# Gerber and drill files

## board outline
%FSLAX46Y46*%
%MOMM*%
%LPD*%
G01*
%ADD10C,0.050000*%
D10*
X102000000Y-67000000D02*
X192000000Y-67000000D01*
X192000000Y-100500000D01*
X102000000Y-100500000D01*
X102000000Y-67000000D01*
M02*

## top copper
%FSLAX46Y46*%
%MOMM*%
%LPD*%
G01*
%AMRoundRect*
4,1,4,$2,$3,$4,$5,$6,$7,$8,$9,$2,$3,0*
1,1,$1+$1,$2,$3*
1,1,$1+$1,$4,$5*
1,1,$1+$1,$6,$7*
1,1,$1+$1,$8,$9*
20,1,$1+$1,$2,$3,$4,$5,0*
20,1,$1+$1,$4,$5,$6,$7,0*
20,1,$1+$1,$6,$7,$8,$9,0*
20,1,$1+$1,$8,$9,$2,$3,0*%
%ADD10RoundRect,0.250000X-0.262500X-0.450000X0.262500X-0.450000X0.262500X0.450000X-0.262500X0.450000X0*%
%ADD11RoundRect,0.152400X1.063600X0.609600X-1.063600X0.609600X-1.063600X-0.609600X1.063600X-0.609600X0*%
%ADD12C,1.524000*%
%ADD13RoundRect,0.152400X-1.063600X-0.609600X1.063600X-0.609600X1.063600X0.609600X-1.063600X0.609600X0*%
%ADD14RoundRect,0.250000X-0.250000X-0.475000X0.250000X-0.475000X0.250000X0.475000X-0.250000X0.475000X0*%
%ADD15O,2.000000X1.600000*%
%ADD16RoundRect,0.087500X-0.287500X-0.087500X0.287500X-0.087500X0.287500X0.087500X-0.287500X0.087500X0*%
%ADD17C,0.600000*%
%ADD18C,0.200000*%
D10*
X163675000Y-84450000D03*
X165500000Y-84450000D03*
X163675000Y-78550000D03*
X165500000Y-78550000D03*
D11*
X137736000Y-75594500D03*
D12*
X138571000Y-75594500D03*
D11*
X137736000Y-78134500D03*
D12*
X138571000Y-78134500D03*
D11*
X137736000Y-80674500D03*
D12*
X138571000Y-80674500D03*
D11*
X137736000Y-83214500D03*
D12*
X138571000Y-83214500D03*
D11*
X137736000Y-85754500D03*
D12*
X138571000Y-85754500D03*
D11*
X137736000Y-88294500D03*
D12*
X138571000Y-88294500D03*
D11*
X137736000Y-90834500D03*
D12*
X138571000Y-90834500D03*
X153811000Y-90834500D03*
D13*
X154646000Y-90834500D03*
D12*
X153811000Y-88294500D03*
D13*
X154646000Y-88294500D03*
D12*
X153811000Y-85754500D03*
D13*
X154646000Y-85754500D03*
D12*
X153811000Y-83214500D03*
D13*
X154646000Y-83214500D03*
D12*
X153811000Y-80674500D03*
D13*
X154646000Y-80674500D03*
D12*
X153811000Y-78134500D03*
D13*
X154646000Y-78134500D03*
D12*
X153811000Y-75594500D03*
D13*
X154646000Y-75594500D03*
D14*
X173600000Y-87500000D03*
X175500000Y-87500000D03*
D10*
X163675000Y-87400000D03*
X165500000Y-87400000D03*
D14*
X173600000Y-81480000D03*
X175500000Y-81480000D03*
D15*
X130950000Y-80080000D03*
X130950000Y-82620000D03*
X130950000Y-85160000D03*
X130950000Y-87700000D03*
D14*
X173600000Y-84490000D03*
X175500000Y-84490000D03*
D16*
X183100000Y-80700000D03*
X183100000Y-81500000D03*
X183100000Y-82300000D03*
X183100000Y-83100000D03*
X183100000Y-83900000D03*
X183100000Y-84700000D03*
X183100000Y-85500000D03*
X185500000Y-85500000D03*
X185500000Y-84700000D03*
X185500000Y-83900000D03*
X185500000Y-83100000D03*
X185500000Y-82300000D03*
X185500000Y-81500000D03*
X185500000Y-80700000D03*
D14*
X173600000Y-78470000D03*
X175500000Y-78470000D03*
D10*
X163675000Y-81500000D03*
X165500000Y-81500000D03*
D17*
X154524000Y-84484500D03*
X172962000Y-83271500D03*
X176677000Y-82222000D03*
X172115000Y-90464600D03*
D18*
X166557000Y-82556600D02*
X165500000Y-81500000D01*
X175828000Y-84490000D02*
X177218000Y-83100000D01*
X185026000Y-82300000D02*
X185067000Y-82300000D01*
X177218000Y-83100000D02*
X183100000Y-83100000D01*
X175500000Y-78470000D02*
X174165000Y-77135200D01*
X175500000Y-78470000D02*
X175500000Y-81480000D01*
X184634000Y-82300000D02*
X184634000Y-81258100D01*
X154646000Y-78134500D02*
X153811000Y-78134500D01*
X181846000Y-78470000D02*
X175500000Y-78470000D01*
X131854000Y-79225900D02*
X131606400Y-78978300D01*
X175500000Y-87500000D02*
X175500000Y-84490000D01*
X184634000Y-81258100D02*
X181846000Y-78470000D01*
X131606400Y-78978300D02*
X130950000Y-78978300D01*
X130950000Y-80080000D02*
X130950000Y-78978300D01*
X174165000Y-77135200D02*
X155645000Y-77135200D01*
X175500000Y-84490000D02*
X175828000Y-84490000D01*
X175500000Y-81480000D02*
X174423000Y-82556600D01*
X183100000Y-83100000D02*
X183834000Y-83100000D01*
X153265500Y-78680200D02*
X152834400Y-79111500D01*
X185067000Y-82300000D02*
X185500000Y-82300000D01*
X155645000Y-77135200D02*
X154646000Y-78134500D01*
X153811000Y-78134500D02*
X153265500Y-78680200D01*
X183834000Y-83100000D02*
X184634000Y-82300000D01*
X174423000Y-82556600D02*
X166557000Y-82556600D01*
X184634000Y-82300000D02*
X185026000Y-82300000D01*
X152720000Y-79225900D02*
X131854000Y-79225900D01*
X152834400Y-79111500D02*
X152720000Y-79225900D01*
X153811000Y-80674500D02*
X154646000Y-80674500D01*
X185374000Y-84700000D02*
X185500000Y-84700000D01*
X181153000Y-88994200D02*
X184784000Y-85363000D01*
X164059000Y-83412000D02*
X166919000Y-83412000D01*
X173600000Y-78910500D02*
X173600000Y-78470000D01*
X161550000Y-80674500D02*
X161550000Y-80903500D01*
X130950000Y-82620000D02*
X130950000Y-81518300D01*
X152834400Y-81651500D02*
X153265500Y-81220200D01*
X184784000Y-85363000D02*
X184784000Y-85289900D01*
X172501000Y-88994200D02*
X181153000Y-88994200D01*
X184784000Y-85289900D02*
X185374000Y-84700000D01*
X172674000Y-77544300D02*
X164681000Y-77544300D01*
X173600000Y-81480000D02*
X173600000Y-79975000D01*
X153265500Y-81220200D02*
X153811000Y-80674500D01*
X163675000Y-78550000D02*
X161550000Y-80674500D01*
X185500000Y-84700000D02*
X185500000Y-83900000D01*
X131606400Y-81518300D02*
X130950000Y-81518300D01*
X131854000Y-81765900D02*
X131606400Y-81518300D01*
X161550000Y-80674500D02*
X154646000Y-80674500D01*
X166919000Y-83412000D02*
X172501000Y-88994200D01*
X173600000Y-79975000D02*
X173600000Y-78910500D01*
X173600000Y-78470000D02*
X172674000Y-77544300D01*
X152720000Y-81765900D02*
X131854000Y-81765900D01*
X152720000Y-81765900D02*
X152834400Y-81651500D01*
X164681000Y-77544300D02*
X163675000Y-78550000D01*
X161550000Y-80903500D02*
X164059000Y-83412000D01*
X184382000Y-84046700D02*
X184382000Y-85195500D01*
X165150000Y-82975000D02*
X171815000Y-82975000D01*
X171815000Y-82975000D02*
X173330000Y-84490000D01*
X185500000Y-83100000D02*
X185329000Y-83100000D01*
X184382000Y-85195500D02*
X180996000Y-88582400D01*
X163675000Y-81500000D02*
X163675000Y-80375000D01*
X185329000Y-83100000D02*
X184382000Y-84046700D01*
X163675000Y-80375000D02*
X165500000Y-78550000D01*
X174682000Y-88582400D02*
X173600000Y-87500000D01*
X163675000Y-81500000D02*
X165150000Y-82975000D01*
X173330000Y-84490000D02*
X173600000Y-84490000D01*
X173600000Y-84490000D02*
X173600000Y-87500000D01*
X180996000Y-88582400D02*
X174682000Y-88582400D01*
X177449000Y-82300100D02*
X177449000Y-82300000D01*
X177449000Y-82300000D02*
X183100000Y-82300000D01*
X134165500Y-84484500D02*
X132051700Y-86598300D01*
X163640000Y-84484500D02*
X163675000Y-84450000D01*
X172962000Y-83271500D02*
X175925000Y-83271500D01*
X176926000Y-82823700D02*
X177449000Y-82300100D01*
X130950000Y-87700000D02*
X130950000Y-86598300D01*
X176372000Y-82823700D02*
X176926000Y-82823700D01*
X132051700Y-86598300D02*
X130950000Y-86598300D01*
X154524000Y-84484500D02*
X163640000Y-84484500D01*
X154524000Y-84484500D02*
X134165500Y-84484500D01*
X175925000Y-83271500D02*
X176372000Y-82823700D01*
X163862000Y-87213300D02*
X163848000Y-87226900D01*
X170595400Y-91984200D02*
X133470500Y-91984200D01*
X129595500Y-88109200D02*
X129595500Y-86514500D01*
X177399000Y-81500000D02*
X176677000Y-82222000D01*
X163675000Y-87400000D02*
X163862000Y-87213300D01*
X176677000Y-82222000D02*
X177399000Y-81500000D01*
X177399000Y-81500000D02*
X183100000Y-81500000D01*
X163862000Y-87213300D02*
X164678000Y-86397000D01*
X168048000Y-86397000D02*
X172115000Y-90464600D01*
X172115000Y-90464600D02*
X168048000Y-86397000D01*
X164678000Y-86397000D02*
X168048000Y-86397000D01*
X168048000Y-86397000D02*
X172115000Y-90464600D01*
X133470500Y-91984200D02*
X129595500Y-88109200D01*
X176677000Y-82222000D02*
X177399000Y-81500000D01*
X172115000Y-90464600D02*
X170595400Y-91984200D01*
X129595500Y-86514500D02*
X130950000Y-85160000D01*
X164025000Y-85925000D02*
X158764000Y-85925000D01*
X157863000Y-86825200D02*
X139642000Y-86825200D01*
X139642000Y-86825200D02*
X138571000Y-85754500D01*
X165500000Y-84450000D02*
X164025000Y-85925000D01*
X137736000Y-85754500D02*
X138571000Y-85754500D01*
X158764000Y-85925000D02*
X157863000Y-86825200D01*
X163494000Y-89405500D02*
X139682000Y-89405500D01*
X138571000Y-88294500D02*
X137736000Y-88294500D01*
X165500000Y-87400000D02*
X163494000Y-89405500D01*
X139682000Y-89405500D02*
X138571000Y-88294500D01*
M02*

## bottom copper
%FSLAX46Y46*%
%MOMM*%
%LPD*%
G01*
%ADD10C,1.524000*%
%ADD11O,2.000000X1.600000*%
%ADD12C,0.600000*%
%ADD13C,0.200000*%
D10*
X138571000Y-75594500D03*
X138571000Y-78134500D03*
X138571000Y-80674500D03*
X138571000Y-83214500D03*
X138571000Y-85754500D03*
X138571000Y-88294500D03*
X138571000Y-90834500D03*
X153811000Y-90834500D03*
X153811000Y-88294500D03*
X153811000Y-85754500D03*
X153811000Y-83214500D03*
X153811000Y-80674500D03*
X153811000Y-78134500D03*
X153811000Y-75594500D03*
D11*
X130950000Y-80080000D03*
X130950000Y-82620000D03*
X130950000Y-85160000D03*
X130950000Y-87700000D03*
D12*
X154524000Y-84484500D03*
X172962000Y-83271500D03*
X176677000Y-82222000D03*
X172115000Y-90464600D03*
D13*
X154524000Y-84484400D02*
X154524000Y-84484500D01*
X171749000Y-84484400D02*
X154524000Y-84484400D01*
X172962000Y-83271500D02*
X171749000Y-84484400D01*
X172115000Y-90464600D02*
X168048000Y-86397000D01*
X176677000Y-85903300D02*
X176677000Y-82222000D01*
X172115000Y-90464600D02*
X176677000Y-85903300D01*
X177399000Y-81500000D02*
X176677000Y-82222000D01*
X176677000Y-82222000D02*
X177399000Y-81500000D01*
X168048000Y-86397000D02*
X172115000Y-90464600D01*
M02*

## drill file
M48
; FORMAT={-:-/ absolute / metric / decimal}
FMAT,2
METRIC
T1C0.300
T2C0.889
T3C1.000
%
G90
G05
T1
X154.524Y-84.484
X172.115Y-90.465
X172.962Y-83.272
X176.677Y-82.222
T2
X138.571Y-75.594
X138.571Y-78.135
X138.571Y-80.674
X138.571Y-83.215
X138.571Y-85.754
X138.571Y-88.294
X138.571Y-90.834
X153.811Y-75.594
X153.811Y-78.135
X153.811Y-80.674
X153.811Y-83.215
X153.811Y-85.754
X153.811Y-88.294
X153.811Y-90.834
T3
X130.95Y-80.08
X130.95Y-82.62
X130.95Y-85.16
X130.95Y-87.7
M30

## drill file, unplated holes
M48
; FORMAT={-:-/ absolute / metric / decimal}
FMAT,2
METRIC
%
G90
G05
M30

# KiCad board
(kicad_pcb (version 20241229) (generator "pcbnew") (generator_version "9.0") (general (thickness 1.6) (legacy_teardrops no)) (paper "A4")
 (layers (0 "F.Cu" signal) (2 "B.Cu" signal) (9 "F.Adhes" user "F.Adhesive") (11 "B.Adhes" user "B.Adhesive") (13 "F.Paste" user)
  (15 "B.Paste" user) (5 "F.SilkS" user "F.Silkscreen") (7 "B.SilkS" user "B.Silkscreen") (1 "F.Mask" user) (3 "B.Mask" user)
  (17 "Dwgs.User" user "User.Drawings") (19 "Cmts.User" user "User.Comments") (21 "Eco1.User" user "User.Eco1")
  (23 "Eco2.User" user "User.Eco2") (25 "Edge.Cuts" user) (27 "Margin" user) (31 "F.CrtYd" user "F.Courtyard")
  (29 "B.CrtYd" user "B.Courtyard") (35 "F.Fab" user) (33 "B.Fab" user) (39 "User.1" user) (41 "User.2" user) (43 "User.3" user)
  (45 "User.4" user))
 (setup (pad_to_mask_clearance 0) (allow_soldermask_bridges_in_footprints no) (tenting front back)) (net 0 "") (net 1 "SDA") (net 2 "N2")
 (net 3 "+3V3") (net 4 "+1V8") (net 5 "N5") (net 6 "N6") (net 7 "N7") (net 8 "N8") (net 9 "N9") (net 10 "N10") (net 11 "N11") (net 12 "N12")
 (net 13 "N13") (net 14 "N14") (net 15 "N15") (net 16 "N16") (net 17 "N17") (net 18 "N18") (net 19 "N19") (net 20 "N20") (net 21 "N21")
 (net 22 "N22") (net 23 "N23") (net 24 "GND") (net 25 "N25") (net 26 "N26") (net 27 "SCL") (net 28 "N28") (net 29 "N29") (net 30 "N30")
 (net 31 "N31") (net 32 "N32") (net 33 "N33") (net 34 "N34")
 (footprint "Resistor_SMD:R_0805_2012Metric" (layer "F.Cu") (at 164.5875 84.45)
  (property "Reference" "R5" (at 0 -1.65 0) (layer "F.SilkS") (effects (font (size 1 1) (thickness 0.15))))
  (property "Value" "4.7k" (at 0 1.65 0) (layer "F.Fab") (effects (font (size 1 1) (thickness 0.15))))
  (pad "1" smd roundrect (at -0.9125 0) (size 1.025 1.4) (layers "F.Cu" "F.Mask" "F.Paste") (roundrect_rratio 0.243902) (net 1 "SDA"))
  (pad "2" smd roundrect (at 0.9125 0) (size 1.025 1.4) (layers "F.Cu" "F.Mask" "F.Paste") (roundrect_rratio 0.243902) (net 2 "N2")))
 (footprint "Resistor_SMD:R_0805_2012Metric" (layer "F.Cu") (at 164.5875 78.55)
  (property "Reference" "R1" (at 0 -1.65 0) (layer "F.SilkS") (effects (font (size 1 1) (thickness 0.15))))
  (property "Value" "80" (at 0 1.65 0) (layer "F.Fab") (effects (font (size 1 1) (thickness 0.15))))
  (pad "1" smd roundrect (at -0.9125 0) (size 1.025 1.4) (layers "F.Cu" "F.Mask" "F.Paste") (roundrect_rratio 0.243902) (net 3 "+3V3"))
  (pad "2" smd roundrect (at 0.9125 0) (size 1.025 1.4) (layers "F.Cu" "F.Mask" "F.Paste") (roundrect_rratio 0.243902) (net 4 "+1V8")))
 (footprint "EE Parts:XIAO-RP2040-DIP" (layer "F.Cu") (at 146.191 83.2145)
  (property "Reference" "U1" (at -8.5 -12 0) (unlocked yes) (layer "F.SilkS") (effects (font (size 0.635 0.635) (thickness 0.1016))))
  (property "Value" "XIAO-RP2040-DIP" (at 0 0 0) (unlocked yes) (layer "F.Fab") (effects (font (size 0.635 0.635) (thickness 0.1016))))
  (pad "1" smd roundrect (at -8.455 -7.62 180) (size 2.432 1.524) (layers "F.Cu" "F.Mask") (roundrect_rratio 0.1) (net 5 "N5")
   (thermal_bridge_angle 45))
  (pad "1" thru_hole circle (at -7.62 -7.62 180) (size 1.524 1.524) (drill 0.889) (layers "*.Cu" "*.Mask") (remove_unused_layers no)
   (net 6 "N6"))
  (pad "2" smd roundrect (at -8.455 -5.08 180) (size 2.432 1.524) (layers "F.Cu" "F.Mask") (roundrect_rratio 0.1) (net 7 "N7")
   (thermal_bridge_angle 45))
  (pad "2" thru_hole circle (at -7.62 -5.08 180) (size 1.524 1.524) (drill 0.889) (layers "*.Cu" "*.Mask") (remove_unused_layers no)
   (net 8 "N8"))
  (pad "3" smd roundrect (at -8.455 -2.54 180) (size 2.432 1.524) (layers "F.Cu" "F.Mask") (roundrect_rratio 0.1) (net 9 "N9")
   (thermal_bridge_angle 45))
  (pad "3" thru_hole circle (at -7.62 -2.54 180) (size 1.524 1.524) (drill 0.889) (layers "*.Cu" "*.Mask") (remove_unused_layers no)
   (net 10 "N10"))
  (pad "4" smd roundrect (at -8.455 0 180) (size 2.432 1.524) (layers "F.Cu" "F.Mask") (roundrect_rratio 0.1) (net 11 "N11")
   (thermal_bridge_angle 45))
  (pad "4" thru_hole circle (at -7.62 0 180) (size 1.524 1.524) (drill 0.889) (layers "*.Cu" "*.Mask") (remove_unused_layers no)
   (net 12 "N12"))
  (pad "5" smd roundrect (at -8.455 2.54 180) (size 2.432 1.524) (layers "F.Cu" "F.Mask") (roundrect_rratio 0.1) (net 2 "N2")
   (thermal_bridge_angle 45))
  (pad "5" thru_hole circle (at -7.62 2.54 180) (size 1.524 1.524) (drill 0.889) (layers "*.Cu" "*.Mask") (remove_unused_layers no)
   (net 2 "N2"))
  (pad "6" smd roundrect (at -8.455 5.08 180) (size 2.432 1.524) (layers "F.Cu" "F.Mask") (roundrect_rratio 0.1) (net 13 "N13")
   (thermal_bridge_angle 45))
  (pad "6" thru_hole circle (at -7.62 5.08 180) (size 1.524 1.524) (drill 0.889) (layers "*.Cu" "*.Mask") (remove_unused_layers no)
   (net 13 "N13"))
  (pad "7" smd roundrect (at -8.455 7.62 180) (size 2.432 1.524) (layers "F.Cu" "F.Mask") (roundrect_rratio 0.1) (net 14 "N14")
   (thermal_bridge_angle 45))
  (pad "7" thru_hole circle (at -7.62 7.62 180) (size 1.524 1.524) (drill 0.889) (layers "*.Cu" "*.Mask") (remove_unused_layers no)
   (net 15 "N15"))
  (pad "8" thru_hole circle (at 7.62 7.62) (size 1.524 1.524) (drill 0.889) (layers "*.Cu" "*.Mask") (remove_unused_layers no)
   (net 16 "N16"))
  (pad "8" smd roundrect (at 8.455 7.62) (size 2.432 1.524) (layers "F.Cu" "F.Mask") (roundrect_rratio 0.1) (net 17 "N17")
   (thermal_bridge_angle 45))
  (pad "9" thru_hole circle (at 7.62 5.08) (size 1.524 1.524) (drill 0.889) (layers "*.Cu" "*.Mask") (remove_unused_layers no)
   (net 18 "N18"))
  (pad "9" smd roundrect (at 8.455 5.08) (size 2.432 1.524) (layers "F.Cu" "F.Mask") (roundrect_rratio 0.1) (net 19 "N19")
   (thermal_bridge_angle 45))
  (pad "10" thru_hole circle (at 7.62 2.54) (size 1.524 1.524) (drill 0.889) (layers "*.Cu" "*.Mask") (remove_unused_layers no)
   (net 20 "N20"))
  (pad "10" smd roundrect (at 8.455 2.54) (size 2.432 1.524) (layers "F.Cu" "F.Mask") (roundrect_rratio 0.1) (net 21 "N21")
   (thermal_bridge_angle 45))
  (pad "11" thru_hole circle (at 7.62 0) (size 1.524 1.524) (drill 0.889) (layers "*.Cu" "*.Mask") (remove_unused_layers no) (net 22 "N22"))
  (pad "11" smd roundrect (at 8.455 0) (size 2.432 1.524) (layers "F.Cu" "F.Mask") (roundrect_rratio 0.1) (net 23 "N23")
   (thermal_bridge_angle 45))
  (pad "12" thru_hole circle (at 7.62 -2.54) (size 1.524 1.524) (drill 0.889) (layers "*.Cu" "*.Mask") (remove_unused_layers no)
   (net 3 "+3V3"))
  (pad "12" smd roundrect (at 8.455 -2.54) (size 2.432 1.524) (layers "F.Cu" "F.Mask") (roundrect_rratio 0.1) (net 3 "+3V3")
   (thermal_bridge_angle 45))
  (pad "13" thru_hole circle (at 7.62 -5.08) (size 1.524 1.524) (drill 0.889) (layers "*.Cu" "*.Mask") (remove_unused_layers no)
   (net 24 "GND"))
  (pad "13" smd roundrect (at 8.455 -5.08) (size 2.432 1.524) (layers "F.Cu" "F.Mask") (roundrect_rratio 0.1) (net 24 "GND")
   (thermal_bridge_angle 45))
  (pad "14" thru_hole circle (at 7.62 -7.62) (size 1.524 1.524) (drill 0.889) (layers "*.Cu" "*.Mask") (remove_unused_layers no)
   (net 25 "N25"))
  (pad "14" smd roundrect (at 8.455 -7.62) (size 2.432 1.524) (layers "F.Cu" "F.Mask") (roundrect_rratio 0.1) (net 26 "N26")
   (thermal_bridge_angle 45)))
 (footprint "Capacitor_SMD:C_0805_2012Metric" (layer "F.Cu") (at 174.55 87.5)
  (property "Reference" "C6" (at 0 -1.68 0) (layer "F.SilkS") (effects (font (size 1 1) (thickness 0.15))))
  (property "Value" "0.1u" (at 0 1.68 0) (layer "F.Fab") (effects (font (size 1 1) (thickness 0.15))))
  (pad "1" smd roundrect (at -0.95 0) (size 1 1.45) (layers "F.Cu" "F.Mask" "F.Paste") (roundrect_rratio 0.25) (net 4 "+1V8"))
  (pad "2" smd roundrect (at 0.95 0) (size 1 1.45) (layers "F.Cu" "F.Mask" "F.Paste") (roundrect_rratio 0.25) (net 24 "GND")))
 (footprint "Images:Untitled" (layer "F.Cu") (at 186.5 95)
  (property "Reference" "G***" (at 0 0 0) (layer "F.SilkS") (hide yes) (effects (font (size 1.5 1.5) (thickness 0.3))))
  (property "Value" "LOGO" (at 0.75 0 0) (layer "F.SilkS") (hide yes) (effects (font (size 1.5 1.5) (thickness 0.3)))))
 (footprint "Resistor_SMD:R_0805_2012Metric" (layer "F.Cu") (at 164.5875 87.4)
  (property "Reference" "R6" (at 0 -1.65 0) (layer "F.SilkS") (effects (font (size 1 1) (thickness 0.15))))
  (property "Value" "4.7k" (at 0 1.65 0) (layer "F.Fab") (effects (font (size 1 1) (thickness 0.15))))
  (pad "1" smd roundrect (at -0.9125 0) (size 1.025 1.4) (layers "F.Cu" "F.Mask" "F.Paste") (roundrect_rratio 0.243902) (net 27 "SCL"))
  (pad "2" smd roundrect (at 0.9125 0) (size 1.025 1.4) (layers "F.Cu" "F.Mask" "F.Paste") (roundrect_rratio 0.243902) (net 13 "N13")))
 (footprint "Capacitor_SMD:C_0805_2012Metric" (layer "F.Cu") (at 174.55 81.48)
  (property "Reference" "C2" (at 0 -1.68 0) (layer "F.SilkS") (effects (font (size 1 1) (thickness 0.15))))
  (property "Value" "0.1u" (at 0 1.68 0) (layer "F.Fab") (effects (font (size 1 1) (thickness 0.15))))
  (pad "1" smd roundrect (at -0.95 0) (size 1 1.45) (layers "F.Cu" "F.Mask" "F.Paste") (roundrect_rratio 0.25) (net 3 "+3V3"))
  (pad "2" smd roundrect (at 0.95 0) (size 1 1.45) (layers "F.Cu" "F.Mask" "F.Paste") (roundrect_rratio 0.25) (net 24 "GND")))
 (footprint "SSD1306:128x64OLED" (layer "F.Cu") (at 120.35 83.7 -90)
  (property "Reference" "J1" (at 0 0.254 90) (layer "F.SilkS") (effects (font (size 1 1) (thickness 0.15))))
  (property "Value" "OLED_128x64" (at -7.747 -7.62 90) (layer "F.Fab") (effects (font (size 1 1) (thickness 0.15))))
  (pad "1" thru_hole oval (at -3.62 -10.6) (size 2 1.6) (drill 1) (layers "*.Cu" "*.Mask") (remove_unused_layers no) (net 24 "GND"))
  (pad "2" thru_hole oval (at -1.08 -10.6) (size 2 1.6) (drill 1) (layers "*.Cu" "*.Mask") (remove_unused_layers no) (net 3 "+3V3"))
  (pad "3" thru_hole oval (at 1.46 -10.6) (size 2 1.6) (drill 1) (layers "*.Cu" "*.Mask") (remove_unused_layers no) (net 27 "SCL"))
  (pad "4" thru_hole oval (at 4 -10.6) (size 2 1.6) (drill 1) (layers "*.Cu" "*.Mask") (remove_unused_layers no) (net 1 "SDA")))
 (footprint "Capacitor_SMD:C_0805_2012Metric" (layer "F.Cu") (at 174.55 84.49)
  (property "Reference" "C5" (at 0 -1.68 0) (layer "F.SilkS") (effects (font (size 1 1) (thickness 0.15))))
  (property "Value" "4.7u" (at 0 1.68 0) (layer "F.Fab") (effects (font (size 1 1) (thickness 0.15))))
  (pad "1" smd roundrect (at -0.95 0) (size 1 1.45) (layers "F.Cu" "F.Mask" "F.Paste") (roundrect_rratio 0.25) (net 4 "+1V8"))
  (pad "2" smd roundrect (at 0.95 0) (size 1 1.45) (layers "F.Cu" "F.Mask" "F.Paste") (roundrect_rratio 0.25) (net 24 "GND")))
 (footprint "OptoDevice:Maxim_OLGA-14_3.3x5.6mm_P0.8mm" (layer "F.Cu") (at 184.3 83.1)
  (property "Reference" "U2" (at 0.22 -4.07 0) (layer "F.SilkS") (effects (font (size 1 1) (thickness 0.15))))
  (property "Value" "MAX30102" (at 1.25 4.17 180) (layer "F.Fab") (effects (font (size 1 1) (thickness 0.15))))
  (pad "1" smd roundrect (at -1.2 -2.4) (size 0.75 0.35) (layers "F.Cu" "F.Mask" "F.Paste") (roundrect_rratio 0.25) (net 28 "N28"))
  (pad "2" smd roundrect (at -1.2 -1.6) (size 0.75 0.35) (layers "F.Cu" "F.Mask" "F.Paste") (roundrect_rratio 0.25) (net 27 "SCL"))
  (pad "3" smd roundrect (at -1.2 -0.8) (size 0.75 0.35) (layers "F.Cu" "F.Mask" "F.Paste") (roundrect_rratio 0.25) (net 1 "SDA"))
  (pad "4" smd roundrect (at -1.2 0) (size 0.75 0.35) (layers "F.Cu" "F.Mask" "F.Paste") (roundrect_rratio 0.25) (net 24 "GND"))
  (pad "5" smd roundrect (at -1.2 0.8) (size 0.75 0.35) (layers "F.Cu" "F.Mask" "F.Paste") (roundrect_rratio 0.25) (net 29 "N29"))
  (pad "6" smd roundrect (at -1.2 1.6) (size 0.75 0.35) (layers "F.Cu" "F.Mask" "F.Paste") (roundrect_rratio 0.25) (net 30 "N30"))
  (pad "7" smd roundrect (at -1.2 2.4) (size 0.75 0.35) (layers "F.Cu" "F.Mask" "F.Paste") (roundrect_rratio 0.25) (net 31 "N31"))
  (pad "8" smd roundrect (at 1.2 2.4) (size 0.75 0.35) (layers "F.Cu" "F.Mask" "F.Paste") (roundrect_rratio 0.25) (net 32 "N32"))
  (pad "9" smd roundrect (at 1.2 1.6) (size 0.75 0.35) (layers "F.Cu" "F.Mask" "F.Paste") (roundrect_rratio 0.25) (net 3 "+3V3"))
  (pad "10" smd roundrect (at 1.2 0.8) (size 0.75 0.35) (layers "F.Cu" "F.Mask" "F.Paste") (roundrect_rratio 0.25) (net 3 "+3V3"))
  (pad "11" smd roundrect (at 1.2 0) (size 0.75 0.35) (layers "F.Cu" "F.Mask" "F.Paste") (roundrect_rratio 0.25) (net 4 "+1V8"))
  (pad "12" smd roundrect (at 1.2 -0.8) (size 0.75 0.35) (layers "F.Cu" "F.Mask" "F.Paste") (roundrect_rratio 0.25) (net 24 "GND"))
  (pad "13" smd roundrect (at 1.2 -1.6) (size 0.75 0.35) (layers "F.Cu" "F.Mask" "F.Paste") (roundrect_rratio 0.25) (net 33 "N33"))
  (pad "14" smd roundrect (at 1.2 -2.4) (size 0.75 0.35) (layers "F.Cu" "F.Mask" "F.Paste") (roundrect_rratio 0.25) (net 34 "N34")))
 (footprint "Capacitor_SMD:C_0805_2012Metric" (layer "F.Cu") (at 174.55 78.47)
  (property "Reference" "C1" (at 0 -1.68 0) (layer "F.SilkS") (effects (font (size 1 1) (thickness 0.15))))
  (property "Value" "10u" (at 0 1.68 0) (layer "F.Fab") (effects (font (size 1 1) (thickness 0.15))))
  (pad "1" smd roundrect (at -0.95 0) (size 1 1.45) (layers "F.Cu" "F.Mask" "F.Paste") (roundrect_rratio 0.25) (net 3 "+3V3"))
  (pad "2" smd roundrect (at 0.95 0) (size 1 1.45) (layers "F.Cu" "F.Mask" "F.Paste") (roundrect_rratio 0.25) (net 24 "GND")))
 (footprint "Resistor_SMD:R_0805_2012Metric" (layer "F.Cu") (at 164.5875 81.5)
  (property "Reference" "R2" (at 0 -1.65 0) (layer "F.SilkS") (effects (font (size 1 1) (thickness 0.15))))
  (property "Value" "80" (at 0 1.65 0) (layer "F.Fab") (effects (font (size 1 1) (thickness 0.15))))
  (pad "1" smd roundrect (at -0.9125 0) (size 1.025 1.4) (layers "F.Cu" "F.Mask" "F.Paste") (roundrect_rratio 0.243902) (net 4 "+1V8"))
  (pad "2" smd roundrect (at 0.9125 0) (size 1.025 1.4) (layers "F.Cu" "F.Mask" "F.Paste") (roundrect_rratio 0.243902) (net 24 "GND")))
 (gr_rect (start 102 67) (end 192 100.5) (stroke (width 0.05) (type default)) (fill no) (layer "Edge.Cuts"))
 (segment (start 166.557 82.5566) (end 165.5 81.5) (width 0.2) (layer "F.Cu") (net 24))
 (segment (start 175.828 84.49) (end 177.218 83.1) (width 0.2) (layer "F.Cu") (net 24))
 (segment (start 185.026 82.3) (end 185.067 82.3) (width 0.2) (layer "F.Cu") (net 24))
 (segment (start 177.218 83.1) (end 183.1 83.1) (width 0.2) (layer "F.Cu") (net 24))
 (segment (start 175.5 78.47) (end 174.165 77.1352) (width 0.2) (layer "F.Cu") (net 24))
 (segment (start 175.5 78.47) (end 175.5 81.48) (width 0.2) (layer "F.Cu") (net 24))
 (segment (start 184.634 82.3) (end 184.634 81.2581) (width 0.2) (layer "F.Cu") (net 24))
 (segment (start 154.646 78.1345) (end 153.811 78.1345) (width 0.2) (layer "F.Cu") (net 24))
 (segment (start 181.846 78.47) (end 175.5 78.47) (width 0.2) (layer "F.Cu") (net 24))
 (segment (start 131.854 79.2259) (end 131.6064 78.9783) (width 0.2) (layer "F.Cu") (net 24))
 (segment (start 175.5 87.5) (end 175.5 84.49) (width 0.2) (layer "F.Cu") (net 24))
 (segment (start 184.634 81.2581) (end 181.846 78.47) (width 0.2) (layer "F.Cu") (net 24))
 (segment (start 131.6064 78.9783) (end 130.95 78.9783) (width 0.2) (layer "F.Cu") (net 24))
 (segment (start 130.95 80.08) (end 130.95 78.9783) (width 0.2) (layer "F.Cu") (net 24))
 (segment (start 174.165 77.1352) (end 155.645 77.1352) (width 0.2) (layer "F.Cu") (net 24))
 (segment (start 175.5 84.49) (end 175.828 84.49) (width 0.2) (layer "F.Cu") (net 24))
 (segment (start 175.5 81.48) (end 174.423 82.5566) (width 0.2) (layer "F.Cu") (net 24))
 (segment (start 183.1 83.1) (end 183.834 83.1) (width 0.2) (layer "F.Cu") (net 24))
 (segment (start 153.2655 78.6802) (end 152.8344 79.1115) (width 0.2) (layer "F.Cu") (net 24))
 (segment (start 185.067 82.3) (end 185.5 82.3) (width 0.2) (layer "F.Cu") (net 24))
 (segment (start 155.645 77.1352) (end 154.646 78.1345) (width 0.2) (layer "F.Cu") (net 24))
 (segment (start 153.811 78.1345) (end 153.2655 78.6802) (width 0.2) (layer "F.Cu") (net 24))
 (segment (start 183.834 83.1) (end 184.634 82.3) (width 0.2) (layer "F.Cu") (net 24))
 (segment (start 174.423 82.5566) (end 166.557 82.5566) (width 0.2) (layer "F.Cu") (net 24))
 (segment (start 184.634 82.3) (end 185.026 82.3) (width 0.2) (layer "F.Cu") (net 24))
 (segment (start 152.72 79.2259) (end 131.854 79.2259) (width 0.2) (layer "F.Cu") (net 24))
 (segment (start 152.8344 79.1115) (end 152.72 79.2259) (width 0.2) (layer "F.Cu") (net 24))
 (segment (start 153.811 80.6745) (end 154.646 80.6745) (width 0.2) (layer "F.Cu") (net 3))
 (segment (start 185.374 84.7) (end 185.5 84.7) (width 0.2) (layer "F.Cu") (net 3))
 (segment (start 181.153 88.9942) (end 184.784 85.363) (width 0.2) (layer "F.Cu") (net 3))
 (segment (start 164.059 83.412) (end 166.919 83.412) (width 0.2) (layer "F.Cu") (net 3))
 (segment (start 173.6 78.9105) (end 173.6 78.47) (width 0.2) (layer "F.Cu") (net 3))
 (segment (start 161.55 80.6745) (end 161.55 80.9035) (width 0.2) (layer "F.Cu") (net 3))
 (segment (start 130.95 82.62) (end 130.95 81.5183) (width 0.2) (layer "F.Cu") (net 3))
 (segment (start 152.8344 81.6515) (end 153.2655 81.2202) (width 0.2) (layer "F.Cu") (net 3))
 (segment (start 184.784 85.363) (end 184.784 85.2899) (width 0.2) (layer "F.Cu") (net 3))
 (segment (start 172.501 88.9942) (end 181.153 88.9942) (width 0.2) (layer "F.Cu") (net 3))
 (segment (start 184.784 85.2899) (end 185.374 84.7) (width 0.2) (layer "F.Cu") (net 3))
 (segment (start 172.674 77.5443) (end 164.681 77.5443) (width 0.2) (layer "F.Cu") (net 3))
 (segment (start 173.6 81.48) (end 173.6 79.975) (width 0.2) (layer "F.Cu") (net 3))
 (segment (start 153.2655 81.2202) (end 153.811 80.6745) (width 0.2) (layer "F.Cu") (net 3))
 (segment (start 163.675 78.55) (end 161.55 80.6745) (width 0.2) (layer "F.Cu") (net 3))
 (segment (start 185.5 84.7) (end 185.5 83.9) (width 0.2) (layer "F.Cu") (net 3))
 (segment (start 131.6064 81.5183) (end 130.95 81.5183) (width 0.2) (layer "F.Cu") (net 3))
 (segment (start 131.854 81.7659) (end 131.6064 81.5183) (width 0.2) (layer "F.Cu") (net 3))
 (segment (start 161.55 80.6745) (end 154.646 80.6745) (width 0.2) (layer "F.Cu") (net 3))
 (segment (start 166.919 83.412) (end 172.501 88.9942) (width 0.2) (layer "F.Cu") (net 3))
 (segment (start 173.6 79.975) (end 173.6 78.9105) (width 0.2) (layer "F.Cu") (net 3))
 (segment (start 173.6 78.47) (end 172.674 77.5443) (width 0.2) (layer "F.Cu") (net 3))
 (segment (start 152.72 81.7659) (end 131.854 81.7659) (width 0.2) (layer "F.Cu") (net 3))
 (segment (start 152.72 81.7659) (end 152.8344 81.6515) (width 0.2) (layer "F.Cu") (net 3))
 (segment (start 164.681 77.5443) (end 163.675 78.55) (width 0.2) (layer "F.Cu") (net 3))
 (segment (start 161.55 80.9035) (end 164.059 83.412) (width 0.2) (layer "F.Cu") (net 3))
 (segment (start 184.382 84.0467) (end 184.382 85.1955) (width 0.2) (layer "F.Cu") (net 4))
 (segment (start 165.15 82.975) (end 171.815 82.975) (width 0.2) (layer "F.Cu") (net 4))
 (segment (start 171.815 82.975) (end 173.33 84.49) (width 0.2) (layer "F.Cu") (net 4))
 (segment (start 185.5 83.1) (end 185.329 83.1) (width 0.2) (layer "F.Cu") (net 4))
 (segment (start 184.382 85.1955) (end 180.996 88.5824) (width 0.2) (layer "F.Cu") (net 4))
 (segment (start 163.675 81.5) (end 163.675 80.375) (width 0.2) (layer "F.Cu") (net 4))
 (segment (start 185.329 83.1) (end 184.382 84.0467) (width 0.2) (layer "F.Cu") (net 4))
 (segment (start 163.675 80.375) (end 165.5 78.55) (width 0.2) (layer "F.Cu") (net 4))
 (segment (start 174.682 88.5824) (end 173.6 87.5) (width 0.2) (layer "F.Cu") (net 4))
 (segment (start 163.675 81.5) (end 165.15 82.975) (width 0.2) (layer "F.Cu") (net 4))
 (segment (start 173.33 84.49) (end 173.6 84.49) (width 0.2) (layer "F.Cu") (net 4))
 (segment (start 173.6 84.49) (end 173.6 87.5) (width 0.2) (layer "F.Cu") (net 4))
 (segment (start 180.996 88.5824) (end 174.682 88.5824) (width 0.2) (layer "F.Cu") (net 4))
 (segment (start 177.449 82.3001) (end 177.449 82.3) (width 0.2) (layer "F.Cu") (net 1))
 (segment (start 177.449 82.3) (end 183.1 82.3) (width 0.2) (layer "F.Cu") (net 1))
 (segment (start 134.1655 84.4845) (end 132.0517 86.5983) (width 0.2) (layer "F.Cu") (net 1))
 (segment (start 163.64 84.4845) (end 163.675 84.45) (width 0.2) (layer "F.Cu") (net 1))
 (segment (start 172.962 83.2715) (end 175.925 83.2715) (width 0.2) (layer "F.Cu") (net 1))
 (segment (start 176.926 82.8237) (end 177.449 82.3001) (width 0.2) (layer "F.Cu") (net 1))
 (segment (start 130.95 87.7) (end 130.95 86.5983) (width 0.2) (layer "F.Cu") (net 1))
 (segment (start 176.372 82.8237) (end 176.926 82.8237) (width 0.2) (layer "F.Cu") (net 1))
 (segment (start 132.0517 86.5983) (end 130.95 86.5983) (width 0.2) (layer "F.Cu") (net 1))
 (segment (start 154.524 84.4845) (end 163.64 84.4845) (width 0.2) (layer "F.Cu") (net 1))
 (segment (start 154.524 84.4845) (end 134.1655 84.4845) (width 0.2) (layer "F.Cu") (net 1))
 (segment (start 175.925 83.2715) (end 176.372 82.8237) (width 0.2) (layer "F.Cu") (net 1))
 (via (at 154.524 84.4845) (size 0.6) (drill 0.3) (layers "F.Cu" "B.Cu") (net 1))
 (via (at 172.962 83.2715) (size 0.6) (drill 0.3) (layers "F.Cu" "B.Cu") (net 1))
 (segment (start 154.524 84.4844) (end 154.524 84.4845) (width 0.2) (layer "B.Cu") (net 1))
 (segment (start 171.749 84.4844) (end 154.524 84.4844) (width 0.2) (layer "B.Cu") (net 1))
 (segment (start 172.962 83.2715) (end 171.749 84.4844) (width 0.2) (layer "B.Cu") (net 1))
 (segment (start 163.862 87.2133) (end 163.848 87.2269) (width 0.2) (layer "F.Cu") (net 27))
 (segment (start 170.5954 91.9842) (end 133.4705 91.9842) (width 0.2) (layer "F.Cu") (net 27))
 (segment (start 129.5955 88.1092) (end 129.5955 86.5145) (width 0.2) (layer "F.Cu") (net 27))
 (segment (start 177.399 81.5) (end 176.677 82.222) (width 0.2) (layer "F.Cu") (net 27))
 (segment (start 163.675 87.4) (end 163.862 87.2133) (width 0.2) (layer "F.Cu") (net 27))
 (segment (start 176.677 82.222) (end 177.399 81.5) (width 0.2) (layer "F.Cu") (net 27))
 (segment (start 177.399 81.5) (end 183.1 81.5) (width 0.2) (layer "F.Cu") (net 27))
 (segment (start 163.862 87.2133) (end 164.678 86.397) (width 0.2) (layer "F.Cu") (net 27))
 (segment (start 168.048 86.397) (end 172.115 90.4646) (width 0.2) (layer "F.Cu") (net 27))
 (segment (start 172.115 90.4646) (end 168.048 86.397) (width 0.2) (layer "F.Cu") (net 27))
 (segment (start 164.678 86.397) (end 168.048 86.397) (width 0.2) (layer "F.Cu") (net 27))
 (segment (start 168.048 86.397) (end 172.115 90.4646) (width 0.2) (layer "F.Cu") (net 27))
 (segment (start 133.4705 91.9842) (end 129.5955 88.1092) (width 0.2) (layer "F.Cu") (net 27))
 (segment (start 176.677 82.222) (end 177.399 81.5) (width 0.2) (layer "F.Cu") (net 27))
 (segment (start 172.115 90.4646) (end 170.5954 91.9842) (width 0.2) (layer "F.Cu") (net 27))
 (segment (start 129.5955 86.5145) (end 130.95 85.16) (width 0.2) (layer "F.Cu") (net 27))
 (via (at 176.677 82.222) (size 0.6) (drill 0.3) (layers "F.Cu" "B.Cu") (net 27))
 (via (at 172.115 90.4646) (size 0.6) (drill 0.3) (layers "F.Cu" "B.Cu") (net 27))
 (segment (start 172.115 90.4646) (end 168.048 86.397) (width 0.2) (layer "B.Cu") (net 27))
 (segment (start 176.677 85.9033) (end 176.677 82.222) (width 0.2) (layer "B.Cu") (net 27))
 (segment (start 172.115 90.4646) (end 176.677 85.9033) (width 0.2) (layer "B.Cu") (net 27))
 (segment (start 177.399 81.5) (end 176.677 82.222) (width 0.2) (layer "B.Cu") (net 27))
 (segment (start 176.677 82.222) (end 177.399 81.5) (width 0.2) (layer "B.Cu") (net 27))
 (segment (start 168.048 86.397) (end 172.115 90.4646) (width 0.2) (layer "B.Cu") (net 27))
 (segment (start 164.025 85.925) (end 158.764 85.925) (width 0.2) (layer "F.Cu") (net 2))
 (segment (start 157.863 86.8252) (end 139.642 86.8252) (width 0.2) (layer "F.Cu") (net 2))
 (segment (start 139.642 86.8252) (end 138.571 85.7545) (width 0.2) (layer "F.Cu") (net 2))
 (segment (start 165.5 84.45) (end 164.025 85.925) (width 0.2) (layer "F.Cu") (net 2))
 (segment (start 137.736 85.7545) (end 138.571 85.7545) (width 0.2) (layer "F.Cu") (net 2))
 (segment (start 158.764 85.925) (end 157.863 86.8252) (width 0.2) (layer "F.Cu") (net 2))
 (segment (start 163.494 89.4055) (end 139.682 89.4055) (width 0.2) (layer "F.Cu") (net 13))
 (segment (start 138.571 88.2945) (end 137.736 88.2945) (width 0.2) (layer "F.Cu") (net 13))
 (segment (start 165.5 87.4) (end 163.494 89.4055) (width 0.2) (layer "F.Cu") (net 13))
 (segment (start 139.682 89.4055) (end 138.571 88.2945) (width 0.2) (layer "F.Cu") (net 13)))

